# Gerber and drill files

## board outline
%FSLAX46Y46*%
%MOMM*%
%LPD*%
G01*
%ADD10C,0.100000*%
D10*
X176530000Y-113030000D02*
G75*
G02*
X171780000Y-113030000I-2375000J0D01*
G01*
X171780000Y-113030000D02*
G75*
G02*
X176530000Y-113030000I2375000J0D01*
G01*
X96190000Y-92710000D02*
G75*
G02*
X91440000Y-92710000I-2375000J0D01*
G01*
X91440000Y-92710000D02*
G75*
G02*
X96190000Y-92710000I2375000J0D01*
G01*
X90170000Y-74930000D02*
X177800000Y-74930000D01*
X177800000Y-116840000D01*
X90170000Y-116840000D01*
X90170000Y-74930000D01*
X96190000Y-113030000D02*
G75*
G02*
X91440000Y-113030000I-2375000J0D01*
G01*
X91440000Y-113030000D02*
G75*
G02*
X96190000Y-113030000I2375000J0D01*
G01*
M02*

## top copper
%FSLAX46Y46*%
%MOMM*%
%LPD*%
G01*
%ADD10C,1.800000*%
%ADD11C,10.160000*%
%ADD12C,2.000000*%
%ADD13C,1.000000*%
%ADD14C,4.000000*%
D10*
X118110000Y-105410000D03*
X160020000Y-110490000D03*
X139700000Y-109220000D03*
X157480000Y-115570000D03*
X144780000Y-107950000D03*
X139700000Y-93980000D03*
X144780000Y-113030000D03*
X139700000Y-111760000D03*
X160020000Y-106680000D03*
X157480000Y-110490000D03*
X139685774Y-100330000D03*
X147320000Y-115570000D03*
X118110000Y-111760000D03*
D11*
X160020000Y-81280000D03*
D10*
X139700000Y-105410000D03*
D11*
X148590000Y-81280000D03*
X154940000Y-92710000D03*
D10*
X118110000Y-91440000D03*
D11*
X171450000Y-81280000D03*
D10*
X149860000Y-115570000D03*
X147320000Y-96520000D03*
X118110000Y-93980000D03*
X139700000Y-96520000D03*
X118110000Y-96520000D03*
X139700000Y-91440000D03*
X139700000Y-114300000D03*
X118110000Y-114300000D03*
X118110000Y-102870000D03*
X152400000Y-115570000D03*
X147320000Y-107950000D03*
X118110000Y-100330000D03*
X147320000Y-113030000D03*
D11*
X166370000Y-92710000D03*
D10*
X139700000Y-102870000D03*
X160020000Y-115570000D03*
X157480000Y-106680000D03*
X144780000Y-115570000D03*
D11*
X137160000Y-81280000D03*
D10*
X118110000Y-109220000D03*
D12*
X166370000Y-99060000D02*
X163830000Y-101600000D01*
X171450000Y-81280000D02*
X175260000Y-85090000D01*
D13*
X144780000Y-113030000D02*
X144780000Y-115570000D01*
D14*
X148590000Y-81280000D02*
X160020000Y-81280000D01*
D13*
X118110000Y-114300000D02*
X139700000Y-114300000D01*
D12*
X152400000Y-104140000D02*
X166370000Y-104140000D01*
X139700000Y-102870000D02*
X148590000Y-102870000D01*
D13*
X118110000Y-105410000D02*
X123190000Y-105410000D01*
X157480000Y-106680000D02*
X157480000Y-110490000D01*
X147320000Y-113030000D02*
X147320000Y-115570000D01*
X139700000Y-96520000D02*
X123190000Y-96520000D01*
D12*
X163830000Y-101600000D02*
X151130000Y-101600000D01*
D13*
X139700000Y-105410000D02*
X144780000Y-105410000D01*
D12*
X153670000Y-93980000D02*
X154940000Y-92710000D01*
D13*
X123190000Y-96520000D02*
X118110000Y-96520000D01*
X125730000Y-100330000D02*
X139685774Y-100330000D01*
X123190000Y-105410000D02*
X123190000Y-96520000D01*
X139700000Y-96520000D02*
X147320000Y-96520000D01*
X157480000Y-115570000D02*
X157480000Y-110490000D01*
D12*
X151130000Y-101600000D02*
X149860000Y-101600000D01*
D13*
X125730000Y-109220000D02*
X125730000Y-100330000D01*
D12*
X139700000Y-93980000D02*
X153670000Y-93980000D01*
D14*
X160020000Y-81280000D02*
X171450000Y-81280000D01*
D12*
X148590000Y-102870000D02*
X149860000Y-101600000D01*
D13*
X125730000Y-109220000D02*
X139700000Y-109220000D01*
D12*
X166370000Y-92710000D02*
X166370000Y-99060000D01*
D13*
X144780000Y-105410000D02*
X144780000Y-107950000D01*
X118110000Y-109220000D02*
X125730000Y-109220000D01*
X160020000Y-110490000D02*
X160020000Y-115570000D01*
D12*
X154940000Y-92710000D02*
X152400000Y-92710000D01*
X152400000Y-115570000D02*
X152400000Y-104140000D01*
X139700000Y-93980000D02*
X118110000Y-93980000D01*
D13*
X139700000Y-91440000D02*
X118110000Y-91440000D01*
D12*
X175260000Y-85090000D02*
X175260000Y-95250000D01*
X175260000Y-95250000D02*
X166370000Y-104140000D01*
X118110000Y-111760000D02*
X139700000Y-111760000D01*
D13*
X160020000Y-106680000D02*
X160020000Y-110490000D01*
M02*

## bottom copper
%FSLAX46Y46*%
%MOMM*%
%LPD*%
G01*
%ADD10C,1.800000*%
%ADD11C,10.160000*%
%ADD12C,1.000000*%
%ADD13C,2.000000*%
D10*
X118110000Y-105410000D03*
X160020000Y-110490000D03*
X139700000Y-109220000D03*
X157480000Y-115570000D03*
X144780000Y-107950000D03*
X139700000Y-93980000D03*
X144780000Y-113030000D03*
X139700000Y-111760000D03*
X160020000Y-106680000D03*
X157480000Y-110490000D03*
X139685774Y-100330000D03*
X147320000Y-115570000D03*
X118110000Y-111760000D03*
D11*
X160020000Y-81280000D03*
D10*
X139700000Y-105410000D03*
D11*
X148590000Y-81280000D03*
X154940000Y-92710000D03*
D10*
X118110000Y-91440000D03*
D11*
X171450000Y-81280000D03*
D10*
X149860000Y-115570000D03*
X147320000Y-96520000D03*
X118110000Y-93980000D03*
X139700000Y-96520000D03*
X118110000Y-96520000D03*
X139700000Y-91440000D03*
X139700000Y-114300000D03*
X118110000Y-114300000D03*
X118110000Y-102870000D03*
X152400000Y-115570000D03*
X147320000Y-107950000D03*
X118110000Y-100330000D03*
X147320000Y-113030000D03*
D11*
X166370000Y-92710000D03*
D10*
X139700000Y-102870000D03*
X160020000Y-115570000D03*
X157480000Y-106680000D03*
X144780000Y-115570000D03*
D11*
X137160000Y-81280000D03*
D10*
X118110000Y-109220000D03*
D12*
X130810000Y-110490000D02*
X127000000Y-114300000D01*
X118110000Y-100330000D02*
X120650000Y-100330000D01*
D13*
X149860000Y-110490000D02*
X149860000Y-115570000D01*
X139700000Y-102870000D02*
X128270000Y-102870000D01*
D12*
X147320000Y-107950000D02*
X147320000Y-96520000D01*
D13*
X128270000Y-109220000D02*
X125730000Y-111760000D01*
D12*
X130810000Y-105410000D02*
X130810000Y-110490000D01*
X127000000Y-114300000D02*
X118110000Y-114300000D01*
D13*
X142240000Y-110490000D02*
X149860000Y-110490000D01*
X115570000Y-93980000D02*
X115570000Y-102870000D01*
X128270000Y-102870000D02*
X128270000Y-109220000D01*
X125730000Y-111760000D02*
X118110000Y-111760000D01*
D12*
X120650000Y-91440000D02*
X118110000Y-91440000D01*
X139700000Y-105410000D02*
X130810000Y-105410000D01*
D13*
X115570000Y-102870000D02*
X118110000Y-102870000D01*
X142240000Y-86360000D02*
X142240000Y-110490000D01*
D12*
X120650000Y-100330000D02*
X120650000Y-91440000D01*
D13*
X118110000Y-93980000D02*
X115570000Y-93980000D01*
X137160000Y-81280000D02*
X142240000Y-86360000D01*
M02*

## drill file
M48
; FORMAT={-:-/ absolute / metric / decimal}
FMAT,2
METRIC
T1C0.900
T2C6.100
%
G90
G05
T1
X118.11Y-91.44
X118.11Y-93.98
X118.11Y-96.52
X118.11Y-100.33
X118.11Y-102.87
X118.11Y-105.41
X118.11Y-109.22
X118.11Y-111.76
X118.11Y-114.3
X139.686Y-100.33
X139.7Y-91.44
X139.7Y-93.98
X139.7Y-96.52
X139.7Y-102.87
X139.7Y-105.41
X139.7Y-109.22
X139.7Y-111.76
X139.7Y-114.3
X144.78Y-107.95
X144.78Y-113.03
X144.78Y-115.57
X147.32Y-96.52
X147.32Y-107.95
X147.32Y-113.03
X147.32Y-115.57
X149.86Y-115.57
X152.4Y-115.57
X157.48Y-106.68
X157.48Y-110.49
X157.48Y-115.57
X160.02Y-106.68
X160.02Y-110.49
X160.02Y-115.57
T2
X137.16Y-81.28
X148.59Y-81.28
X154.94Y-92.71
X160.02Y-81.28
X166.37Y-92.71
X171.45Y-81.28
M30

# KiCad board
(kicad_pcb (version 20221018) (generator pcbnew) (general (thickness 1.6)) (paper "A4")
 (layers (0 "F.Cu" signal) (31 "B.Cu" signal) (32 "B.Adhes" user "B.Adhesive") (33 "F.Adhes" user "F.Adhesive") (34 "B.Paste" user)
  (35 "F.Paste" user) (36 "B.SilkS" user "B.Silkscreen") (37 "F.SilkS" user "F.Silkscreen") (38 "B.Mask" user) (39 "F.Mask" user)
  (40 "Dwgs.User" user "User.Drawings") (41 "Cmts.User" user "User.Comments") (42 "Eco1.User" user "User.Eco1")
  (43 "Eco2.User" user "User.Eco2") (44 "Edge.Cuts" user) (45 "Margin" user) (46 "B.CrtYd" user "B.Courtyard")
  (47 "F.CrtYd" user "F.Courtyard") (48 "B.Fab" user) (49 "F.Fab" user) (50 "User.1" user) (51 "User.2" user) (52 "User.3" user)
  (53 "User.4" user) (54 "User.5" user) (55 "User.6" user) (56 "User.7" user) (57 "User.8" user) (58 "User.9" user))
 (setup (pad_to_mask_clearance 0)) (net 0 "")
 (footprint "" (layer "F.Cu") (at 118.11 105.41)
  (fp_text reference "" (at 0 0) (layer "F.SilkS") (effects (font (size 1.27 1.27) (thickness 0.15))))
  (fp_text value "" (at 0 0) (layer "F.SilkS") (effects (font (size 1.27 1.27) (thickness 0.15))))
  (pad "1" thru_hole circle (at 0 0) (size 1.8 1.8) (drill 0.9) (layers "*.Cu" "*.Mask")))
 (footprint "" (layer "F.Cu") (at 160.02 110.49)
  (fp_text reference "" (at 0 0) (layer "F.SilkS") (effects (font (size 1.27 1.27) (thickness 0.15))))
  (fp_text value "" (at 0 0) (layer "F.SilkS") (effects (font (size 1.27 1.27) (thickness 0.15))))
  (pad "1" thru_hole circle (at 0 0) (size 1.8 1.8) (drill 0.9) (layers "*.Cu" "*.Mask")))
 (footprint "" (layer "F.Cu") (at 139.7 109.22)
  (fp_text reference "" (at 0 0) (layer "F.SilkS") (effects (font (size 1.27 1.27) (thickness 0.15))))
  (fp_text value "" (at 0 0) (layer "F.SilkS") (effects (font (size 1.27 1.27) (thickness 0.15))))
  (pad "1" thru_hole circle (at 0 0) (size 1.8 1.8) (drill 0.9) (layers "*.Cu" "*.Mask")))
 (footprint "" (layer "F.Cu") (at 157.48 115.57)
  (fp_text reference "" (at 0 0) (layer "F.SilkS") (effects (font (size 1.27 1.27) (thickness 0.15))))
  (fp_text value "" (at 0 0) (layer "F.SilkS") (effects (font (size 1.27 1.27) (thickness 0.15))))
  (pad "1" thru_hole circle (at 0 0) (size 1.8 1.8) (drill 0.9) (layers "*.Cu" "*.Mask")))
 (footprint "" (layer "F.Cu") (at 144.78 107.95)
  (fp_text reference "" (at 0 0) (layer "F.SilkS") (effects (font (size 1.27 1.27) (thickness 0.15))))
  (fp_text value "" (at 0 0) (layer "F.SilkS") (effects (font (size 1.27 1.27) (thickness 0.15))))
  (pad "1" thru_hole circle (at 0 0) (size 1.8 1.8) (drill 0.9) (layers "*.Cu" "*.Mask")))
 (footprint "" (layer "F.Cu") (at 139.7 93.98)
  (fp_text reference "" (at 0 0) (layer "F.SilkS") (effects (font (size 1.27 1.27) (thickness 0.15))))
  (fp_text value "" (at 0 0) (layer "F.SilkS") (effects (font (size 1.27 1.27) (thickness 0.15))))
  (pad "1" thru_hole circle (at 0 0) (size 1.8 1.8) (drill 0.9) (layers "*.Cu" "*.Mask")))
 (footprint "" (layer "F.Cu") (at 144.78 113.03)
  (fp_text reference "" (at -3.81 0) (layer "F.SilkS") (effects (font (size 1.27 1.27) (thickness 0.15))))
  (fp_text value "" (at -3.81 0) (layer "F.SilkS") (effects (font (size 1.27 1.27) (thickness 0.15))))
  (pad "1" thru_hole circle (at 0 0) (size 1.8 1.8) (drill 0.9) (layers "*.Cu" "*.Mask")))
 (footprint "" (layer "F.Cu") (at 139.7 111.76)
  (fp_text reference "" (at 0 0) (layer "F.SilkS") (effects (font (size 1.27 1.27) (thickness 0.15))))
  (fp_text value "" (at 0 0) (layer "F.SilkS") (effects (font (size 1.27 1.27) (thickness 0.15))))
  (pad "1" thru_hole circle (at 0 0) (size 1.8 1.8) (drill 0.9) (layers "*.Cu" "*.Mask")))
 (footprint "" (layer "F.Cu") (at 160.02 106.68)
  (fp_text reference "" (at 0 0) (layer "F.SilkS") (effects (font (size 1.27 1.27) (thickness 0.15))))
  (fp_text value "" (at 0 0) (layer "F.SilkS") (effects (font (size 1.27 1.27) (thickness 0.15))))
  (pad "1" thru_hole circle (at 0 0) (size 1.8 1.8) (drill 0.9) (layers "*.Cu" "*.Mask")))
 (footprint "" (layer "F.Cu") (at 157.48 110.49)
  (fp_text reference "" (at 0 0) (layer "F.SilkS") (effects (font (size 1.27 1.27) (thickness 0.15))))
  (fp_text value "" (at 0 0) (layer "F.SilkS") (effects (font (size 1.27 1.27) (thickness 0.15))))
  (pad "1" thru_hole circle (at 0 0) (size 1.8 1.8) (drill 0.9) (layers "*.Cu" "*.Mask")))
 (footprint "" (layer "F.Cu") (at 139.685774 100.33)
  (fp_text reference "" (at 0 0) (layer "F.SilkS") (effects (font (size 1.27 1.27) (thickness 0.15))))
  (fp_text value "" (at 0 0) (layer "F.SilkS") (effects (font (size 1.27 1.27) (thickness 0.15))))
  (pad "1" thru_hole circle (at 0 0) (size 1.8 1.8) (drill 0.9) (layers "*.Cu" "*.Mask")))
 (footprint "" (layer "F.Cu") (at 147.32 115.57)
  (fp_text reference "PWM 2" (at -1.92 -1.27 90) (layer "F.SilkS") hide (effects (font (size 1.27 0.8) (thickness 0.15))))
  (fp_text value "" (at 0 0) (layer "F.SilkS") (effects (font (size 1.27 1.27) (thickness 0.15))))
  (pad "1" thru_hole circle (at 0 0) (size 1.8 1.8) (drill 0.9) (layers "*.Cu" "*.Mask")))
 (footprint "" (layer "F.Cu") (at 118.11 111.76)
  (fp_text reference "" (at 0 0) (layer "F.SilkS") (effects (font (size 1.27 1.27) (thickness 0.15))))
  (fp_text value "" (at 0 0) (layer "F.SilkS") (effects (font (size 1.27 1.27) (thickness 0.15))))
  (pad "1" thru_hole circle (at 0 0) (size 1.8 1.8) (drill 0.9) (layers "*.Cu" "*.Mask")))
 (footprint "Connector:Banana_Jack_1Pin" (layer "F.Cu") (at 160.02 81.28)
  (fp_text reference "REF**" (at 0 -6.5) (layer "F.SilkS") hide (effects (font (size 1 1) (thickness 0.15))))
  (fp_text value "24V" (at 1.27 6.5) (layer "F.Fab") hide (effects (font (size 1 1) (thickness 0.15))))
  (pad "1" thru_hole circle (at 0 0) (size 10.16 10.16) (drill 6.1) (layers "*.Cu" "*.Mask")))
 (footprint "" (layer "F.Cu") (at 139.7 105.41)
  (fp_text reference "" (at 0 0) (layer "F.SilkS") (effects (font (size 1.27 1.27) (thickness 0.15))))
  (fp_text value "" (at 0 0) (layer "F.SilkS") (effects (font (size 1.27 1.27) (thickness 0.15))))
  (pad "1" thru_hole circle (at 0 0) (size 1.8 1.8) (drill 0.9) (layers "*.Cu" "*.Mask")))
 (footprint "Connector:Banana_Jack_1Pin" (layer "F.Cu") (at 148.59 81.28)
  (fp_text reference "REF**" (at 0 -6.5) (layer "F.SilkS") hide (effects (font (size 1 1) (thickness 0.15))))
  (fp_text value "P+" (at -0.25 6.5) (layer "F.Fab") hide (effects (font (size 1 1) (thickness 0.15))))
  (pad "1" thru_hole circle (at 0 0) (size 10.16 10.16) (drill 6.1) (layers "*.Cu" "*.Mask")))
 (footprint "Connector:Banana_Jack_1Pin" (layer "F.Cu") (at 154.94 92.71)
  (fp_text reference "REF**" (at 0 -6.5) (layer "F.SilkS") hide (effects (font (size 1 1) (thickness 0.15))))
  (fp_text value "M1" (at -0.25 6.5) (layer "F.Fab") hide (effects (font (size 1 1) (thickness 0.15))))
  (pad "1" thru_hole circle (at 0 0) (size 10.16 10.16) (drill 6.1) (layers "*.Cu" "*.Mask")))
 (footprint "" (layer "F.Cu") (at 118.11 91.44)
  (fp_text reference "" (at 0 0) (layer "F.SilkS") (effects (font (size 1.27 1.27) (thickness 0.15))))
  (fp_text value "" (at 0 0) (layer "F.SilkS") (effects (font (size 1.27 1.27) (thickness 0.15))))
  (pad "1" thru_hole circle (at 0 0) (size 1.8 1.8) (drill 0.9) (layers "*.Cu" "*.Mask")))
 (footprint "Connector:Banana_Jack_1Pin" (layer "F.Cu") (at 171.45 81.28)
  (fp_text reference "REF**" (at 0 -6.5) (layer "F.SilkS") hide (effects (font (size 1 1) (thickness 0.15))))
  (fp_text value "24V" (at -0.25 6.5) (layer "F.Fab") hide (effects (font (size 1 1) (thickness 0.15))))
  (pad "1" thru_hole circle (at 0 0) (size 10.16 10.16) (drill 6.1) (layers "*.Cu" "*.Mask")))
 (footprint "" (layer "F.Cu") (at 149.86 115.57)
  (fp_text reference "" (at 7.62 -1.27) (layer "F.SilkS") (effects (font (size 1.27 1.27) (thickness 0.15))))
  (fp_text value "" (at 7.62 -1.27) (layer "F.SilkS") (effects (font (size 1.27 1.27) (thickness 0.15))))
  (pad "1" thru_hole circle (at 0 0) (size 1.8 1.8) (drill 0.9) (layers "*.Cu" "*.Mask")))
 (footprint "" (layer "F.Cu") (at 147.32 96.52)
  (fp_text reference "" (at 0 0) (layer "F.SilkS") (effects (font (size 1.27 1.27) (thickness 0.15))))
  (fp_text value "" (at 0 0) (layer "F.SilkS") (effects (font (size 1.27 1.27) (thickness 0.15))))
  (pad "1" thru_hole circle (at 0 0) (size 1.8 1.8) (drill 0.9) (layers "*.Cu" "*.Mask")))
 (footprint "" (layer "F.Cu") (at 118.11 93.98)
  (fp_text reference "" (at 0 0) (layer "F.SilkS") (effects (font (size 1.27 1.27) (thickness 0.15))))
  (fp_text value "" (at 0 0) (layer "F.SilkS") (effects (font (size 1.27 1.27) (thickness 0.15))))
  (pad "1" thru_hole circle (at 0 0) (size 1.8 1.8) (drill 0.9) (layers "*.Cu" "*.Mask")))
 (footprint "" (layer "F.Cu") (at 139.7 96.52)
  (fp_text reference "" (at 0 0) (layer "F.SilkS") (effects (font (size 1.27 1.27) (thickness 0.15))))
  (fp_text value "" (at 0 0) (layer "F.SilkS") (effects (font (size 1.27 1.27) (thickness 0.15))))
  (pad "1" thru_hole circle (at 0 0) (size 1.8 1.8) (drill 0.9) (layers "*.Cu" "*.Mask")))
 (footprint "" (layer "F.Cu") (at 118.11 96.52)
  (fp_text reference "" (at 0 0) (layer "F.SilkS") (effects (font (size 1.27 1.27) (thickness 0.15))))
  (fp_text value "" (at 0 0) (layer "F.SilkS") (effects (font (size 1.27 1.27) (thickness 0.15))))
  (pad "1" thru_hole circle (at 0 0) (size 1.8 1.8) (drill 0.9) (layers "*.Cu" "*.Mask")))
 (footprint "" (layer "F.Cu") (at 139.7 91.44)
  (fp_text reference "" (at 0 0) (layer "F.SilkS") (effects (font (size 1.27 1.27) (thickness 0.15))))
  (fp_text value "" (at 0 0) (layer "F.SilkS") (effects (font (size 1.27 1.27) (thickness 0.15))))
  (pad "1" thru_hole circle (at 0 0) (size 1.8 1.8) (drill 0.9) (layers "*.Cu" "*.Mask")))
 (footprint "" (layer "F.Cu") (at 139.7 114.3)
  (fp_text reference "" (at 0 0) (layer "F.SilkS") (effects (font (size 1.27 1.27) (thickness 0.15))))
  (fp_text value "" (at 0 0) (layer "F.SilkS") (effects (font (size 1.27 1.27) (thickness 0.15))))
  (pad "1" thru_hole circle (at 0 0) (size 1.8 1.8) (drill 0.9) (layers "*.Cu" "*.Mask")))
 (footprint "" (layer "F.Cu") (at 118.11 114.3)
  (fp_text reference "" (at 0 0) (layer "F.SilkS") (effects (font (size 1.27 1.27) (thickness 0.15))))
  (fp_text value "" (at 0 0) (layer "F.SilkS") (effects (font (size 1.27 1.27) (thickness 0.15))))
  (pad "1" thru_hole circle (at 0 0) (size 1.8 1.8) (drill 0.9) (layers "*.Cu" "*.Mask")))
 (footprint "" (layer "F.Cu") (at 118.11 102.87)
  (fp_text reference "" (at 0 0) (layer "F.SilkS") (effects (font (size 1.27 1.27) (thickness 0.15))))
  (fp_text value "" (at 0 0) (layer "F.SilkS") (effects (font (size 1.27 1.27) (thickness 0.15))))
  (pad "1" thru_hole circle (at 0 0) (size 1.8 1.8) (drill 0.9) (layers "*.Cu" "*.Mask")))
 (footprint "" (layer "F.Cu") (at 152.4 115.57)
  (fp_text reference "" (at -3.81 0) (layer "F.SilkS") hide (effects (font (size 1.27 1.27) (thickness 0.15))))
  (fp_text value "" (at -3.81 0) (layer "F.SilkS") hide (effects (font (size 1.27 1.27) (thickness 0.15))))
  (pad "1" thru_hole circle (at 0 0) (size 1.8 1.8) (drill 0.9) (layers "*.Cu" "*.Mask")))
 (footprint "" (layer "F.Cu") (at 147.32 107.95)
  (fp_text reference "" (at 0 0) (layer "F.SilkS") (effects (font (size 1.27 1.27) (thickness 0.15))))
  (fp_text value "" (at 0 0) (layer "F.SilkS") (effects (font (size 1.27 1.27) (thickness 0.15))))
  (pad "1" thru_hole circle (at 0 0) (size 1.8 1.8) (drill 0.9) (layers "*.Cu" "*.Mask")))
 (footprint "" (layer "F.Cu") (at 118.11 100.33)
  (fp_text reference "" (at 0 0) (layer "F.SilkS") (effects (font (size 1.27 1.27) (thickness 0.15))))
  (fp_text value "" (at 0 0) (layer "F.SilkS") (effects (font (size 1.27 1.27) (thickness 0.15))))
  (pad "1" thru_hole circle (at 0 0) (size 1.8 1.8) (drill 0.9) (layers "*.Cu" "*.Mask")))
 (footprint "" (layer "F.Cu") (at 147.32 113.03)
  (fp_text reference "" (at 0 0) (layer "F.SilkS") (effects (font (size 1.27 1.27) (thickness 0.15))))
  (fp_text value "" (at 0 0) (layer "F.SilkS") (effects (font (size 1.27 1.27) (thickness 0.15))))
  (pad "1" thru_hole circle (at 0 0) (size 1.8 1.8) (drill 0.9) (layers "*.Cu" "*.Mask")))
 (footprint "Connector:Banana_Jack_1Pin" (layer "F.Cu") (at 166.37 92.71)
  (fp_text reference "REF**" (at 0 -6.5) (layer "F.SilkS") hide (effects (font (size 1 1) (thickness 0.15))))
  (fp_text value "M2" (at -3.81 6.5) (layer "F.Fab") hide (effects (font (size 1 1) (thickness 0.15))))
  (pad "1" thru_hole circle (at 0 0) (size 10.16 10.16) (drill 6.1) (layers "*.Cu" "*.Mask")))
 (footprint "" (layer "F.Cu") (at 139.7 102.87)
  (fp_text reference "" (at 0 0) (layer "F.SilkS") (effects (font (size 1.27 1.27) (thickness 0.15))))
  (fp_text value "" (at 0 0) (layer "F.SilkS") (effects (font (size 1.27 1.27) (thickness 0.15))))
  (pad "1" thru_hole circle (at 0 0) (size 1.8 1.8) (drill 0.9) (layers "*.Cu" "*.Mask")))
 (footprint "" (layer "F.Cu") (at 160.02 115.57)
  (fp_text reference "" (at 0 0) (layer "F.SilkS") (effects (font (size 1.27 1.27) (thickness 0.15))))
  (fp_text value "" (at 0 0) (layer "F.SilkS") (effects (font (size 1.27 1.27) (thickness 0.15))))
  (pad "1" thru_hole circle (at 0 0) (size 1.8 1.8) (drill 0.9) (layers "*.Cu" "*.Mask")))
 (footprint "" (layer "F.Cu") (at 157.48 106.68)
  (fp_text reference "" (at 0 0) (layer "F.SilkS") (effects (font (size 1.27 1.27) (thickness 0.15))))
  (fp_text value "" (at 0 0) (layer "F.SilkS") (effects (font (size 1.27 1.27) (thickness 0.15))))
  (pad "1" thru_hole circle (at 0 0) (size 1.8 1.8) (drill 0.9) (layers "*.Cu" "*.Mask")))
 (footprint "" (layer "F.Cu") (at 144.78 115.57)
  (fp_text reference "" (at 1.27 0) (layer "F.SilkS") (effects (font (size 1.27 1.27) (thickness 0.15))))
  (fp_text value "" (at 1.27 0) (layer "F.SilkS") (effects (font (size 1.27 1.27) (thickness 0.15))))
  (pad "1" thru_hole circle (at 0 0) (size 1.8 1.8) (drill 0.9) (layers "*.Cu" "*.Mask")))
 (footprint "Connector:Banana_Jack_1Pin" (layer "F.Cu") (at 137.16 81.28)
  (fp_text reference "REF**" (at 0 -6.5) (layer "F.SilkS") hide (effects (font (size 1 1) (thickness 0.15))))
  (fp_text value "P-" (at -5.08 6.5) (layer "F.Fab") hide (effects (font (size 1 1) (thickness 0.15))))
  (pad "1" thru_hole circle (at 0 0) (size 10.16 10.16) (drill 6.1) (layers "*.Cu" "*.Mask")))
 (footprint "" (layer "F.Cu") (at 118.11 109.22)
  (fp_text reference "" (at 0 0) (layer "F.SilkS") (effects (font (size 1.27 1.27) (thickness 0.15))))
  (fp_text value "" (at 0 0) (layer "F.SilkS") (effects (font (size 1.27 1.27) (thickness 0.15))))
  (pad "1" thru_hole circle (at 0 0) (size 1.8 1.8) (drill 0.9) (layers "*.Cu" "*.Mask")))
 (gr_circle (center 174.155 113.03) (end 176.53 113.03) (stroke (width 0.1) (type default)) (fill none) (layer "Edge.Cuts"))
 (gr_circle (center 93.815 92.71) (end 96.19 92.71) (stroke (width 0.1) (type default)) (fill none) (layer "Edge.Cuts"))
 (gr_rect (start 90.17 74.93) (end 177.8 116.84) (stroke (width 0.1) (type default)) (fill none) (layer "Edge.Cuts"))
 (gr_circle (center 93.815 113.03) (end 96.19 113.03) (stroke (width 0.1) (type default)) (fill none) (layer "Edge.Cuts"))
 (segment (start 166.37 99.06) (end 163.83 101.6) (width 2) (layer "F.Cu") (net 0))
 (segment (start 171.45 81.28) (end 175.26 85.09) (width 2) (layer "F.Cu") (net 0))
 (segment (start 144.78 113.03) (end 144.78 115.57) (width 1) (layer "F.Cu") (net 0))
 (segment (start 148.59 81.28) (end 160.02 81.28) (width 4) (layer "F.Cu") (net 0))
 (segment (start 118.11 114.3) (end 139.7 114.3) (width 1) (layer "F.Cu") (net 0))
 (segment (start 152.4 104.14) (end 166.37 104.14) (width 2) (layer "F.Cu") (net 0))
 (segment (start 139.7 102.87) (end 148.59 102.87) (width 2) (layer "F.Cu") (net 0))
 (segment (start 118.11 105.41) (end 123.19 105.41) (width 1) (layer "F.Cu") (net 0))
 (segment (start 157.48 106.68) (end 157.48 110.49) (width 1) (layer "F.Cu") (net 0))
 (segment (start 147.32 113.03) (end 147.32 115.57) (width 1) (layer "F.Cu") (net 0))
 (segment (start 139.7 96.52) (end 123.19 96.52) (width 1) (layer "F.Cu") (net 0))
 (segment (start 163.83 101.6) (end 151.13 101.6) (width 2) (layer "F.Cu") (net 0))
 (segment (start 139.7 105.41) (end 144.78 105.41) (width 1) (layer "F.Cu") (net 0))
 (segment (start 153.67 93.98) (end 154.94 92.71) (width 2) (layer "F.Cu") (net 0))
 (segment (start 123.19 96.52) (end 118.11 96.52) (width 1) (layer "F.Cu") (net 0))
 (segment (start 125.73 100.33) (end 139.685774 100.33) (width 1) (layer "F.Cu") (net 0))
 (segment (start 123.19 105.41) (end 123.19 96.52) (width 1) (layer "F.Cu") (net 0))
 (segment (start 139.7 96.52) (end 147.32 96.52) (width 1) (layer "F.Cu") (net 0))
 (segment (start 157.48 115.57) (end 157.48 110.49) (width 1) (layer "F.Cu") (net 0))
 (segment (start 151.13 101.6) (end 149.86 101.6) (width 2) (layer "F.Cu") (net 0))
 (segment (start 125.73 109.22) (end 125.73 100.33) (width 1) (layer "F.Cu") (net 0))
 (segment (start 139.7 93.98) (end 153.67 93.98) (width 2) (layer "F.Cu") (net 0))
 (segment (start 160.02 81.28) (end 171.45 81.28) (width 4) (layer "F.Cu") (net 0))
 (segment (start 148.59 102.87) (end 149.86 101.6) (width 2) (layer "F.Cu") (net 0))
 (segment (start 125.73 109.22) (end 139.7 109.22) (width 1) (layer "F.Cu") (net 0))
 (segment (start 166.37 92.71) (end 166.37 99.06) (width 2) (layer "F.Cu") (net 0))
 (segment (start 144.78 105.41) (end 144.78 107.95) (width 1) (layer "F.Cu") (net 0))
 (segment (start 118.11 109.22) (end 125.73 109.22) (width 1) (layer "F.Cu") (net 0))
 (segment (start 160.02 110.49) (end 160.02 115.57) (width 1) (layer "F.Cu") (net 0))
 (segment (start 154.94 92.71) (end 152.4 92.71) (width 2) (layer "F.Cu") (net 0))
 (segment (start 152.4 115.57) (end 152.4 104.14) (width 2) (layer "F.Cu") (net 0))
 (segment (start 139.7 93.98) (end 118.11 93.98) (width 2) (layer "F.Cu") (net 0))
 (segment (start 139.7 91.44) (end 118.11 91.44) (width 1) (layer "F.Cu") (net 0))
 (segment (start 175.26 85.09) (end 175.26 95.25) (width 2) (layer "F.Cu") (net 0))
 (segment (start 175.26 95.25) (end 166.37 104.14) (width 2) (layer "F.Cu") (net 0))
 (segment (start 118.11 111.76) (end 139.7 111.76) (width 2) (layer "F.Cu") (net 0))
 (segment (start 160.02 106.68) (end 160.02 110.49) (width 1) (layer "F.Cu") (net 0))
 (segment (start 130.81 110.49) (end 127 114.3) (width 1) (layer "B.Cu") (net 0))
 (segment (start 118.11 100.33) (end 120.65 100.33) (width 1) (layer "B.Cu") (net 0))
 (segment (start 149.86 110.49) (end 149.86 115.57) (width 2) (layer "B.Cu") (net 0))
 (segment (start 139.7 102.87) (end 128.27 102.87) (width 2) (layer "B.Cu") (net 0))
 (segment (start 147.32 107.95) (end 147.32 96.52) (width 1) (layer "B.Cu") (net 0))
 (segment (start 128.27 109.22) (end 125.73 111.76) (width 2) (layer "B.Cu") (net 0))
 (segment (start 130.81 105.41) (end 130.81 110.49) (width 1) (layer "B.Cu") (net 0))
 (segment (start 127 114.3) (end 118.11 114.3) (width 1) (layer "B.Cu") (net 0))
 (segment (start 142.24 110.49) (end 149.86 110.49) (width 2) (layer "B.Cu") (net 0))
 (segment (start 115.57 93.98) (end 115.57 102.87) (width 2) (layer "B.Cu") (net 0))
 (segment (start 128.27 102.87) (end 128.27 109.22) (width 2) (layer "B.Cu") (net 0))
 (segment (start 125.73 111.76) (end 118.11 111.76) (width 2) (layer "B.Cu") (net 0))
 (segment (start 120.65 91.44) (end 118.11 91.44) (width 1) (layer "B.Cu") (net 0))
 (segment (start 139.7 105.41) (end 130.81 105.41) (width 1) (layer "B.Cu") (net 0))
 (segment (start 115.57 102.87) (end 118.11 102.87) (width 2) (layer "B.Cu") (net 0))
 (segment (start 142.24 86.36) (end 142.24 110.49) (width 2) (layer "B.Cu") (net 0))
 (segment (start 120.65 100.33) (end 120.65 91.44) (width 1) (layer "B.Cu") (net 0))
 (segment (start 118.11 93.98) (end 115.57 93.98) (width 2) (layer "B.Cu") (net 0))
 (segment (start 137.16 81.28) (end 142.24 86.36) (width 2) (layer "B.Cu") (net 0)))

